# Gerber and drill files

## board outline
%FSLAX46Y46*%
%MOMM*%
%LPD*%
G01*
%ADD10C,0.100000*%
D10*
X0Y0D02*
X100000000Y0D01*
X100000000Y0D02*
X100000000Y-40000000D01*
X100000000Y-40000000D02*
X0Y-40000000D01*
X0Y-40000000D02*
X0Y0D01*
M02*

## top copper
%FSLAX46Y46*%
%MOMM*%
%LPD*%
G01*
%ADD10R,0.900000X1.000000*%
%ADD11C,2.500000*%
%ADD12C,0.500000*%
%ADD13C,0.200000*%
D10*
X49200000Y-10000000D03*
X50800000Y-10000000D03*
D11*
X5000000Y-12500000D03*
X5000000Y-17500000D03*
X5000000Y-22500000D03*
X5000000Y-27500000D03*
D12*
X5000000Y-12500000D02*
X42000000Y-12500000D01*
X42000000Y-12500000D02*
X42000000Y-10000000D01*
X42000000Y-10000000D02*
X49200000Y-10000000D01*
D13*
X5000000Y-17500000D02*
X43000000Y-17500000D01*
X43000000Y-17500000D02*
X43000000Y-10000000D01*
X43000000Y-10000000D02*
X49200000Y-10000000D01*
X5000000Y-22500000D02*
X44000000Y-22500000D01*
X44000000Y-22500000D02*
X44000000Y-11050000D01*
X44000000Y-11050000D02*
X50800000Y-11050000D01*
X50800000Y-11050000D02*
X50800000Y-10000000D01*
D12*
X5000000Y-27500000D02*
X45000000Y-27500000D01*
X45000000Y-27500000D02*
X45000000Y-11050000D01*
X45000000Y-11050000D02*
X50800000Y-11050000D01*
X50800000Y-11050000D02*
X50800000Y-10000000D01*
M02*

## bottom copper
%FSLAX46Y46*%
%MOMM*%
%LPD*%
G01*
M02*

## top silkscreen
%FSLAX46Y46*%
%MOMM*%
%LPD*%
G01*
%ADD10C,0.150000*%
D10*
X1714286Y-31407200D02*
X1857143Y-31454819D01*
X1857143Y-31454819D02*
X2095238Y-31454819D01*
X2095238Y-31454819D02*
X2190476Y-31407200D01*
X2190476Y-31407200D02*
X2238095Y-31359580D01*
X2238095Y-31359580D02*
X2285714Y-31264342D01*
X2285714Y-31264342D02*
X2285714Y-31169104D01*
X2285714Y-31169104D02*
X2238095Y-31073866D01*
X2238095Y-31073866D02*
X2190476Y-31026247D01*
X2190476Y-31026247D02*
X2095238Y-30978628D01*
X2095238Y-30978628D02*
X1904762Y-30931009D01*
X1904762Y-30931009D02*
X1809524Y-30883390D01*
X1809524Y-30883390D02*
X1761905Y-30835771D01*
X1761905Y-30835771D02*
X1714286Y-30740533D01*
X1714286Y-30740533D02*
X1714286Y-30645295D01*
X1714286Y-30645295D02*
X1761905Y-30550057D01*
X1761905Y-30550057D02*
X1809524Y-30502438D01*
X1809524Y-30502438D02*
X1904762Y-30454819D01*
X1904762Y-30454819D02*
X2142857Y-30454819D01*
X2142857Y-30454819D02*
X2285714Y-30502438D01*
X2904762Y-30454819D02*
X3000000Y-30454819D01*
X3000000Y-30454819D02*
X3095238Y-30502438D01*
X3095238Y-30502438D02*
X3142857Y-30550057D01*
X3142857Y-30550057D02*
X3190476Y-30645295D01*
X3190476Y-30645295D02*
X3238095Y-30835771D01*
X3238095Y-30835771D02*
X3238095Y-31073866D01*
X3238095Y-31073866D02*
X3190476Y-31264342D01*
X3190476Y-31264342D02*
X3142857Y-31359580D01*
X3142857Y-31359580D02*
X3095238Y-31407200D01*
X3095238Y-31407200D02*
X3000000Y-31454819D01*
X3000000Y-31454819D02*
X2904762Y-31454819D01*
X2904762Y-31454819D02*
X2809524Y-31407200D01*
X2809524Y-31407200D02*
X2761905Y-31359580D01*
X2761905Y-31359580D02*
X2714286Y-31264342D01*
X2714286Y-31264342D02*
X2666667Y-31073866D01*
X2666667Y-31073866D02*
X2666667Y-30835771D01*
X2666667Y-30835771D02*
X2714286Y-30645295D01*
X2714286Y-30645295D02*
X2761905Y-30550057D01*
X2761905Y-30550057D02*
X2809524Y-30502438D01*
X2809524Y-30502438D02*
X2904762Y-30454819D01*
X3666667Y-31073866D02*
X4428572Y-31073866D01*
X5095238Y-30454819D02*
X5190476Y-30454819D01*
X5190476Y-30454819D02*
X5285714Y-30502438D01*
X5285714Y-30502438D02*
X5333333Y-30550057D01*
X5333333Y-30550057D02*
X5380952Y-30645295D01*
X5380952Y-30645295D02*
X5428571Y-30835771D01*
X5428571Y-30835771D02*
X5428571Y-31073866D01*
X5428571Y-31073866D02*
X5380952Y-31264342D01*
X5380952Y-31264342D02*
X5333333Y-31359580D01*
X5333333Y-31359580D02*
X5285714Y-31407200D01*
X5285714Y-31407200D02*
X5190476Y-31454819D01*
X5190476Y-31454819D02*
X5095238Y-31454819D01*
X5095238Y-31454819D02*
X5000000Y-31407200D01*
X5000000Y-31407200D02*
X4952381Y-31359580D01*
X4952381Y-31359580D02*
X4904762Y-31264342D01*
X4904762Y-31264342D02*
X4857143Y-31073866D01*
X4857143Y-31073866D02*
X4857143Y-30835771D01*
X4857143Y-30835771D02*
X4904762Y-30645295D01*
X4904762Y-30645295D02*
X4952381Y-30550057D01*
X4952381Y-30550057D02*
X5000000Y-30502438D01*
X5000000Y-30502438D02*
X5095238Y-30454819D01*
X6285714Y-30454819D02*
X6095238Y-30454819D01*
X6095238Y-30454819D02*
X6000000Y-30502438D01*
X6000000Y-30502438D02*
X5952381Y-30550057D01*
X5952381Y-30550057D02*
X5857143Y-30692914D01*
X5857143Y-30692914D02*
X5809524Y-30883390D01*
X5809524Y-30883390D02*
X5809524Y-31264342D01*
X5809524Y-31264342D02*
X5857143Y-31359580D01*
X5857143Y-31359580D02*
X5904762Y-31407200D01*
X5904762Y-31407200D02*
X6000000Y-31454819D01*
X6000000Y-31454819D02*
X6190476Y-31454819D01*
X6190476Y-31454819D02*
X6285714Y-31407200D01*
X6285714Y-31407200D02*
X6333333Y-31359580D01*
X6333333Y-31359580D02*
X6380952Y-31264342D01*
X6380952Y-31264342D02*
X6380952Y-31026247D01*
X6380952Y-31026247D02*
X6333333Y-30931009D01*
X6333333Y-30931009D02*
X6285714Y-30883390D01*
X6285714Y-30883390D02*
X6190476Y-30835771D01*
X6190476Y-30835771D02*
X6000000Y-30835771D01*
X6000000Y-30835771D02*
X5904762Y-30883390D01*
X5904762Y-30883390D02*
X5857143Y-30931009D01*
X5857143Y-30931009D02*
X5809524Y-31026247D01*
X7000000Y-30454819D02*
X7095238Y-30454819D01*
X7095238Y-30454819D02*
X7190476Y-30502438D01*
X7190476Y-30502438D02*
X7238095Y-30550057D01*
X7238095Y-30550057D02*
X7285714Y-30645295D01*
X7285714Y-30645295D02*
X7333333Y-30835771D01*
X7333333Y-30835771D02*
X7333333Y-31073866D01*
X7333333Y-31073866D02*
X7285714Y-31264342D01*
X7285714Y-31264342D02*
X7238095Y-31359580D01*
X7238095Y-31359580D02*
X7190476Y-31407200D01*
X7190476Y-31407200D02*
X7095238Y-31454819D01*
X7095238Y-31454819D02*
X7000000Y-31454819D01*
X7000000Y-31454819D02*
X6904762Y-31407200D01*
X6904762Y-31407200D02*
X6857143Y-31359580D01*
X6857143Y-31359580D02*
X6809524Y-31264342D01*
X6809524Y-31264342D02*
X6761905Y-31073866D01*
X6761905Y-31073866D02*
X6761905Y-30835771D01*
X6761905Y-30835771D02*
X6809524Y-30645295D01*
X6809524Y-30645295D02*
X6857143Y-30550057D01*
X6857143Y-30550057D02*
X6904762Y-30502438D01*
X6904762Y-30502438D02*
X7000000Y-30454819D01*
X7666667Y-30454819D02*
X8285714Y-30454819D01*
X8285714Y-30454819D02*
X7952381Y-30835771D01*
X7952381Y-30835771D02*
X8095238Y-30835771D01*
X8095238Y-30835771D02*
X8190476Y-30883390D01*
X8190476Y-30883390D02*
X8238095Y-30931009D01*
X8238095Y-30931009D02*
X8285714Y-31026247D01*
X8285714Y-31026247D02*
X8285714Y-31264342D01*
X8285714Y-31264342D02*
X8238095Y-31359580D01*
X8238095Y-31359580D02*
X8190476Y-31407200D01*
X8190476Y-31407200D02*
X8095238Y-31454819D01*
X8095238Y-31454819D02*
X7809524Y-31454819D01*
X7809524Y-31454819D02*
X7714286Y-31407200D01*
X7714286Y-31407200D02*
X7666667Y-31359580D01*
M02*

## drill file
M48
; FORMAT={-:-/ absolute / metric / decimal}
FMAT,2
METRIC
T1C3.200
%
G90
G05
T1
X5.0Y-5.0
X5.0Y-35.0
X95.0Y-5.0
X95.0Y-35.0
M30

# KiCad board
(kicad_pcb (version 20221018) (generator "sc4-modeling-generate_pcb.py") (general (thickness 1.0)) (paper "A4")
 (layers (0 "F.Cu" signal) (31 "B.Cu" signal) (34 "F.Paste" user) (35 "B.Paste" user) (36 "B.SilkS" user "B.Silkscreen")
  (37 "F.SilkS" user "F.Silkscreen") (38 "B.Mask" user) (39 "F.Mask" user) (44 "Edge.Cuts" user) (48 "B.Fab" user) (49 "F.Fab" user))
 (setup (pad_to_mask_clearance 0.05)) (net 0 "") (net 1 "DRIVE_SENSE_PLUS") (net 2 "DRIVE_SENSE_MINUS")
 (gr_line (start 0.0 0.0) (end 100.0 0.0) (layer "Edge.Cuts") (width 0.1))
 (gr_line (start 100.0 0.0) (end 100.0 40.0) (layer "Edge.Cuts") (width 0.1))
 (gr_line (start 100.0 40.0) (end 0.0 40.0) (layer "Edge.Cuts") (width 0.1))
 (gr_line (start 0.0 40.0) (end 0.0 0.0) (layer "Edge.Cuts") (width 0.1))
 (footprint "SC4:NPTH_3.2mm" (layer "F.Cu") (at 5.0 5.0)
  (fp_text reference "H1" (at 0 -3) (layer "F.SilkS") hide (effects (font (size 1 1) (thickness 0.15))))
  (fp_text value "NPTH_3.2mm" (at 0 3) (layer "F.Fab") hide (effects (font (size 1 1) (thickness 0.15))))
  (pad "1" np_thru_hole circle (at 0 0) (size 3.2 3.2) (drill 3.2) (layers "*.Cu" "*.Mask")))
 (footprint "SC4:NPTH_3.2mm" (layer "F.Cu") (at 95.0 5.0)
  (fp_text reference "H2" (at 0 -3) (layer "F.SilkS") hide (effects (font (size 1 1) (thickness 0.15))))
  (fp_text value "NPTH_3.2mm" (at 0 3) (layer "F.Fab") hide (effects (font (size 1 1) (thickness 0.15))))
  (pad "1" np_thru_hole circle (at 0 0) (size 3.2 3.2) (drill 3.2) (layers "*.Cu" "*.Mask")))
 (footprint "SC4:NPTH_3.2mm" (layer "F.Cu") (at 5.0 35.0)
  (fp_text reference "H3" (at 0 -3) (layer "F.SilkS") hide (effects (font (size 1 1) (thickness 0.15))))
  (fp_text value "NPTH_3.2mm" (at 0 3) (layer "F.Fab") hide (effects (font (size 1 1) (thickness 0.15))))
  (pad "1" np_thru_hole circle (at 0 0) (size 3.2 3.2) (drill 3.2) (layers "*.Cu" "*.Mask")))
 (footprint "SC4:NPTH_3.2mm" (layer "F.Cu") (at 95.0 35.0)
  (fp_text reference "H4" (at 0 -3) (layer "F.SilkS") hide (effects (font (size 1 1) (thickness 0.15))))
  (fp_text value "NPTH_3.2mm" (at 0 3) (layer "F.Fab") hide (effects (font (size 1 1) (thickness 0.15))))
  (pad "1" np_thru_hole circle (at 0 0) (size 3.2 3.2) (drill 3.2) (layers "*.Cu" "*.Mask")))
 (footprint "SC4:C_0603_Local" (layer "F.Cu") (at 50.0 10.0 0)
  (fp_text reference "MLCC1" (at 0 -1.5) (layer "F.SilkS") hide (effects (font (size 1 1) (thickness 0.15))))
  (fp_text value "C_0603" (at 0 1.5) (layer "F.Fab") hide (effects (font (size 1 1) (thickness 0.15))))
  (pad "1" smd rect (at -0.8 0) (size 0.9 1.0) (layers "F.Cu" "F.Paste" "F.Mask") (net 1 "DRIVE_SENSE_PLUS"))
  (pad "2" smd rect (at 0.8 0) (size 0.9 1.0) (layers "F.Cu" "F.Paste" "F.Mask") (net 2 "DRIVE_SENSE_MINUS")))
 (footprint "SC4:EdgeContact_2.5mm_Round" (layer "F.Cu") (at 5.0 12.5)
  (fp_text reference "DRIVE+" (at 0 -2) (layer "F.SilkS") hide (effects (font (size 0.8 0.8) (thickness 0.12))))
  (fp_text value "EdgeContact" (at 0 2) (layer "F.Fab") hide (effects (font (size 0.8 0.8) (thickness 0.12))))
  (pad "1" smd circle (at 0 0) (size 2.5 2.5) (layers "F.Cu" "F.Mask") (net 1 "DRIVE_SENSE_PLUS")))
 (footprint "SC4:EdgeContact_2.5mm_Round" (layer "F.Cu") (at 5.0 17.5)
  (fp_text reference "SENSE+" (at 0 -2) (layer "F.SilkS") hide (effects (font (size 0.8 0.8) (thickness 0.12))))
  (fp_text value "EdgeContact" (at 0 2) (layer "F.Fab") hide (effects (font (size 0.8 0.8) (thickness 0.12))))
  (pad "1" smd circle (at 0 0) (size 2.5 2.5) (layers "F.Cu" "F.Mask") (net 1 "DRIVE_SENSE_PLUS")))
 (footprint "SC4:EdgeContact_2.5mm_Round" (layer "F.Cu") (at 5.0 22.5)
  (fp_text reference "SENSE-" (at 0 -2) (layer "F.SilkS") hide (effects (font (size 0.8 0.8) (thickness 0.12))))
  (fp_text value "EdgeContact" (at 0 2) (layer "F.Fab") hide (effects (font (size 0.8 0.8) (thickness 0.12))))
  (pad "1" smd circle (at 0 0) (size 2.5 2.5) (layers "F.Cu" "F.Mask") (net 2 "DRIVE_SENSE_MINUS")))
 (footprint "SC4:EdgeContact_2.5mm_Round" (layer "F.Cu") (at 5.0 27.5)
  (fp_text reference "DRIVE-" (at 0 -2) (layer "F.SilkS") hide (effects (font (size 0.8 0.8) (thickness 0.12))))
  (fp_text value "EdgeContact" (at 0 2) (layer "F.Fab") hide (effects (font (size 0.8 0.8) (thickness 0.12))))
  (pad "1" smd circle (at 0 0) (size 2.5 2.5) (layers "F.Cu" "F.Mask") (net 2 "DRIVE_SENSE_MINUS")))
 (segment (start 5.0 12.5) (end 42.0 12.5) (width 0.5) (layer "F.Cu") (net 1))
 (segment (start 42.0 12.5) (end 42.0 10.0) (width 0.5) (layer "F.Cu") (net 1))
 (segment (start 42.0 10.0) (end 49.2 10.0) (width 0.5) (layer "F.Cu") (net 1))
 (segment (start 5.0 17.5) (end 43.0 17.5) (width 0.2) (layer "F.Cu") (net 1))
 (segment (start 43.0 17.5) (end 43.0 10.0) (width 0.2) (layer "F.Cu") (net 1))
 (segment (start 43.0 10.0) (end 49.2 10.0) (width 0.2) (layer "F.Cu") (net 1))
 (segment (start 5.0 22.5) (end 44.0 22.5) (width 0.2) (layer "F.Cu") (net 2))
 (segment (start 44.0 22.5) (end 44.0 11.05) (width 0.2) (layer "F.Cu") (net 2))
 (segment (start 44.0 11.05) (end 50.8 11.05) (width 0.2) (layer "F.Cu") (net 2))
 (segment (start 50.8 11.05) (end 50.8 10.0) (width 0.2) (layer "F.Cu") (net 2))
 (segment (start 5.0 27.5) (end 45.0 27.5) (width 0.5) (layer "F.Cu") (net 2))
 (segment (start 45.0 27.5) (end 45.0 11.05) (width 0.5) (layer "F.Cu") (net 2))
 (segment (start 45.0 11.05) (end 50.8 11.05) (width 0.5) (layer "F.Cu") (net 2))
 (segment (start 50.8 11.05) (end 50.8 10.0) (width 0.5) (layer "F.Cu") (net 2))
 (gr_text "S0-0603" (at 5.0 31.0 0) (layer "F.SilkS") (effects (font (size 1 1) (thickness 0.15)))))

